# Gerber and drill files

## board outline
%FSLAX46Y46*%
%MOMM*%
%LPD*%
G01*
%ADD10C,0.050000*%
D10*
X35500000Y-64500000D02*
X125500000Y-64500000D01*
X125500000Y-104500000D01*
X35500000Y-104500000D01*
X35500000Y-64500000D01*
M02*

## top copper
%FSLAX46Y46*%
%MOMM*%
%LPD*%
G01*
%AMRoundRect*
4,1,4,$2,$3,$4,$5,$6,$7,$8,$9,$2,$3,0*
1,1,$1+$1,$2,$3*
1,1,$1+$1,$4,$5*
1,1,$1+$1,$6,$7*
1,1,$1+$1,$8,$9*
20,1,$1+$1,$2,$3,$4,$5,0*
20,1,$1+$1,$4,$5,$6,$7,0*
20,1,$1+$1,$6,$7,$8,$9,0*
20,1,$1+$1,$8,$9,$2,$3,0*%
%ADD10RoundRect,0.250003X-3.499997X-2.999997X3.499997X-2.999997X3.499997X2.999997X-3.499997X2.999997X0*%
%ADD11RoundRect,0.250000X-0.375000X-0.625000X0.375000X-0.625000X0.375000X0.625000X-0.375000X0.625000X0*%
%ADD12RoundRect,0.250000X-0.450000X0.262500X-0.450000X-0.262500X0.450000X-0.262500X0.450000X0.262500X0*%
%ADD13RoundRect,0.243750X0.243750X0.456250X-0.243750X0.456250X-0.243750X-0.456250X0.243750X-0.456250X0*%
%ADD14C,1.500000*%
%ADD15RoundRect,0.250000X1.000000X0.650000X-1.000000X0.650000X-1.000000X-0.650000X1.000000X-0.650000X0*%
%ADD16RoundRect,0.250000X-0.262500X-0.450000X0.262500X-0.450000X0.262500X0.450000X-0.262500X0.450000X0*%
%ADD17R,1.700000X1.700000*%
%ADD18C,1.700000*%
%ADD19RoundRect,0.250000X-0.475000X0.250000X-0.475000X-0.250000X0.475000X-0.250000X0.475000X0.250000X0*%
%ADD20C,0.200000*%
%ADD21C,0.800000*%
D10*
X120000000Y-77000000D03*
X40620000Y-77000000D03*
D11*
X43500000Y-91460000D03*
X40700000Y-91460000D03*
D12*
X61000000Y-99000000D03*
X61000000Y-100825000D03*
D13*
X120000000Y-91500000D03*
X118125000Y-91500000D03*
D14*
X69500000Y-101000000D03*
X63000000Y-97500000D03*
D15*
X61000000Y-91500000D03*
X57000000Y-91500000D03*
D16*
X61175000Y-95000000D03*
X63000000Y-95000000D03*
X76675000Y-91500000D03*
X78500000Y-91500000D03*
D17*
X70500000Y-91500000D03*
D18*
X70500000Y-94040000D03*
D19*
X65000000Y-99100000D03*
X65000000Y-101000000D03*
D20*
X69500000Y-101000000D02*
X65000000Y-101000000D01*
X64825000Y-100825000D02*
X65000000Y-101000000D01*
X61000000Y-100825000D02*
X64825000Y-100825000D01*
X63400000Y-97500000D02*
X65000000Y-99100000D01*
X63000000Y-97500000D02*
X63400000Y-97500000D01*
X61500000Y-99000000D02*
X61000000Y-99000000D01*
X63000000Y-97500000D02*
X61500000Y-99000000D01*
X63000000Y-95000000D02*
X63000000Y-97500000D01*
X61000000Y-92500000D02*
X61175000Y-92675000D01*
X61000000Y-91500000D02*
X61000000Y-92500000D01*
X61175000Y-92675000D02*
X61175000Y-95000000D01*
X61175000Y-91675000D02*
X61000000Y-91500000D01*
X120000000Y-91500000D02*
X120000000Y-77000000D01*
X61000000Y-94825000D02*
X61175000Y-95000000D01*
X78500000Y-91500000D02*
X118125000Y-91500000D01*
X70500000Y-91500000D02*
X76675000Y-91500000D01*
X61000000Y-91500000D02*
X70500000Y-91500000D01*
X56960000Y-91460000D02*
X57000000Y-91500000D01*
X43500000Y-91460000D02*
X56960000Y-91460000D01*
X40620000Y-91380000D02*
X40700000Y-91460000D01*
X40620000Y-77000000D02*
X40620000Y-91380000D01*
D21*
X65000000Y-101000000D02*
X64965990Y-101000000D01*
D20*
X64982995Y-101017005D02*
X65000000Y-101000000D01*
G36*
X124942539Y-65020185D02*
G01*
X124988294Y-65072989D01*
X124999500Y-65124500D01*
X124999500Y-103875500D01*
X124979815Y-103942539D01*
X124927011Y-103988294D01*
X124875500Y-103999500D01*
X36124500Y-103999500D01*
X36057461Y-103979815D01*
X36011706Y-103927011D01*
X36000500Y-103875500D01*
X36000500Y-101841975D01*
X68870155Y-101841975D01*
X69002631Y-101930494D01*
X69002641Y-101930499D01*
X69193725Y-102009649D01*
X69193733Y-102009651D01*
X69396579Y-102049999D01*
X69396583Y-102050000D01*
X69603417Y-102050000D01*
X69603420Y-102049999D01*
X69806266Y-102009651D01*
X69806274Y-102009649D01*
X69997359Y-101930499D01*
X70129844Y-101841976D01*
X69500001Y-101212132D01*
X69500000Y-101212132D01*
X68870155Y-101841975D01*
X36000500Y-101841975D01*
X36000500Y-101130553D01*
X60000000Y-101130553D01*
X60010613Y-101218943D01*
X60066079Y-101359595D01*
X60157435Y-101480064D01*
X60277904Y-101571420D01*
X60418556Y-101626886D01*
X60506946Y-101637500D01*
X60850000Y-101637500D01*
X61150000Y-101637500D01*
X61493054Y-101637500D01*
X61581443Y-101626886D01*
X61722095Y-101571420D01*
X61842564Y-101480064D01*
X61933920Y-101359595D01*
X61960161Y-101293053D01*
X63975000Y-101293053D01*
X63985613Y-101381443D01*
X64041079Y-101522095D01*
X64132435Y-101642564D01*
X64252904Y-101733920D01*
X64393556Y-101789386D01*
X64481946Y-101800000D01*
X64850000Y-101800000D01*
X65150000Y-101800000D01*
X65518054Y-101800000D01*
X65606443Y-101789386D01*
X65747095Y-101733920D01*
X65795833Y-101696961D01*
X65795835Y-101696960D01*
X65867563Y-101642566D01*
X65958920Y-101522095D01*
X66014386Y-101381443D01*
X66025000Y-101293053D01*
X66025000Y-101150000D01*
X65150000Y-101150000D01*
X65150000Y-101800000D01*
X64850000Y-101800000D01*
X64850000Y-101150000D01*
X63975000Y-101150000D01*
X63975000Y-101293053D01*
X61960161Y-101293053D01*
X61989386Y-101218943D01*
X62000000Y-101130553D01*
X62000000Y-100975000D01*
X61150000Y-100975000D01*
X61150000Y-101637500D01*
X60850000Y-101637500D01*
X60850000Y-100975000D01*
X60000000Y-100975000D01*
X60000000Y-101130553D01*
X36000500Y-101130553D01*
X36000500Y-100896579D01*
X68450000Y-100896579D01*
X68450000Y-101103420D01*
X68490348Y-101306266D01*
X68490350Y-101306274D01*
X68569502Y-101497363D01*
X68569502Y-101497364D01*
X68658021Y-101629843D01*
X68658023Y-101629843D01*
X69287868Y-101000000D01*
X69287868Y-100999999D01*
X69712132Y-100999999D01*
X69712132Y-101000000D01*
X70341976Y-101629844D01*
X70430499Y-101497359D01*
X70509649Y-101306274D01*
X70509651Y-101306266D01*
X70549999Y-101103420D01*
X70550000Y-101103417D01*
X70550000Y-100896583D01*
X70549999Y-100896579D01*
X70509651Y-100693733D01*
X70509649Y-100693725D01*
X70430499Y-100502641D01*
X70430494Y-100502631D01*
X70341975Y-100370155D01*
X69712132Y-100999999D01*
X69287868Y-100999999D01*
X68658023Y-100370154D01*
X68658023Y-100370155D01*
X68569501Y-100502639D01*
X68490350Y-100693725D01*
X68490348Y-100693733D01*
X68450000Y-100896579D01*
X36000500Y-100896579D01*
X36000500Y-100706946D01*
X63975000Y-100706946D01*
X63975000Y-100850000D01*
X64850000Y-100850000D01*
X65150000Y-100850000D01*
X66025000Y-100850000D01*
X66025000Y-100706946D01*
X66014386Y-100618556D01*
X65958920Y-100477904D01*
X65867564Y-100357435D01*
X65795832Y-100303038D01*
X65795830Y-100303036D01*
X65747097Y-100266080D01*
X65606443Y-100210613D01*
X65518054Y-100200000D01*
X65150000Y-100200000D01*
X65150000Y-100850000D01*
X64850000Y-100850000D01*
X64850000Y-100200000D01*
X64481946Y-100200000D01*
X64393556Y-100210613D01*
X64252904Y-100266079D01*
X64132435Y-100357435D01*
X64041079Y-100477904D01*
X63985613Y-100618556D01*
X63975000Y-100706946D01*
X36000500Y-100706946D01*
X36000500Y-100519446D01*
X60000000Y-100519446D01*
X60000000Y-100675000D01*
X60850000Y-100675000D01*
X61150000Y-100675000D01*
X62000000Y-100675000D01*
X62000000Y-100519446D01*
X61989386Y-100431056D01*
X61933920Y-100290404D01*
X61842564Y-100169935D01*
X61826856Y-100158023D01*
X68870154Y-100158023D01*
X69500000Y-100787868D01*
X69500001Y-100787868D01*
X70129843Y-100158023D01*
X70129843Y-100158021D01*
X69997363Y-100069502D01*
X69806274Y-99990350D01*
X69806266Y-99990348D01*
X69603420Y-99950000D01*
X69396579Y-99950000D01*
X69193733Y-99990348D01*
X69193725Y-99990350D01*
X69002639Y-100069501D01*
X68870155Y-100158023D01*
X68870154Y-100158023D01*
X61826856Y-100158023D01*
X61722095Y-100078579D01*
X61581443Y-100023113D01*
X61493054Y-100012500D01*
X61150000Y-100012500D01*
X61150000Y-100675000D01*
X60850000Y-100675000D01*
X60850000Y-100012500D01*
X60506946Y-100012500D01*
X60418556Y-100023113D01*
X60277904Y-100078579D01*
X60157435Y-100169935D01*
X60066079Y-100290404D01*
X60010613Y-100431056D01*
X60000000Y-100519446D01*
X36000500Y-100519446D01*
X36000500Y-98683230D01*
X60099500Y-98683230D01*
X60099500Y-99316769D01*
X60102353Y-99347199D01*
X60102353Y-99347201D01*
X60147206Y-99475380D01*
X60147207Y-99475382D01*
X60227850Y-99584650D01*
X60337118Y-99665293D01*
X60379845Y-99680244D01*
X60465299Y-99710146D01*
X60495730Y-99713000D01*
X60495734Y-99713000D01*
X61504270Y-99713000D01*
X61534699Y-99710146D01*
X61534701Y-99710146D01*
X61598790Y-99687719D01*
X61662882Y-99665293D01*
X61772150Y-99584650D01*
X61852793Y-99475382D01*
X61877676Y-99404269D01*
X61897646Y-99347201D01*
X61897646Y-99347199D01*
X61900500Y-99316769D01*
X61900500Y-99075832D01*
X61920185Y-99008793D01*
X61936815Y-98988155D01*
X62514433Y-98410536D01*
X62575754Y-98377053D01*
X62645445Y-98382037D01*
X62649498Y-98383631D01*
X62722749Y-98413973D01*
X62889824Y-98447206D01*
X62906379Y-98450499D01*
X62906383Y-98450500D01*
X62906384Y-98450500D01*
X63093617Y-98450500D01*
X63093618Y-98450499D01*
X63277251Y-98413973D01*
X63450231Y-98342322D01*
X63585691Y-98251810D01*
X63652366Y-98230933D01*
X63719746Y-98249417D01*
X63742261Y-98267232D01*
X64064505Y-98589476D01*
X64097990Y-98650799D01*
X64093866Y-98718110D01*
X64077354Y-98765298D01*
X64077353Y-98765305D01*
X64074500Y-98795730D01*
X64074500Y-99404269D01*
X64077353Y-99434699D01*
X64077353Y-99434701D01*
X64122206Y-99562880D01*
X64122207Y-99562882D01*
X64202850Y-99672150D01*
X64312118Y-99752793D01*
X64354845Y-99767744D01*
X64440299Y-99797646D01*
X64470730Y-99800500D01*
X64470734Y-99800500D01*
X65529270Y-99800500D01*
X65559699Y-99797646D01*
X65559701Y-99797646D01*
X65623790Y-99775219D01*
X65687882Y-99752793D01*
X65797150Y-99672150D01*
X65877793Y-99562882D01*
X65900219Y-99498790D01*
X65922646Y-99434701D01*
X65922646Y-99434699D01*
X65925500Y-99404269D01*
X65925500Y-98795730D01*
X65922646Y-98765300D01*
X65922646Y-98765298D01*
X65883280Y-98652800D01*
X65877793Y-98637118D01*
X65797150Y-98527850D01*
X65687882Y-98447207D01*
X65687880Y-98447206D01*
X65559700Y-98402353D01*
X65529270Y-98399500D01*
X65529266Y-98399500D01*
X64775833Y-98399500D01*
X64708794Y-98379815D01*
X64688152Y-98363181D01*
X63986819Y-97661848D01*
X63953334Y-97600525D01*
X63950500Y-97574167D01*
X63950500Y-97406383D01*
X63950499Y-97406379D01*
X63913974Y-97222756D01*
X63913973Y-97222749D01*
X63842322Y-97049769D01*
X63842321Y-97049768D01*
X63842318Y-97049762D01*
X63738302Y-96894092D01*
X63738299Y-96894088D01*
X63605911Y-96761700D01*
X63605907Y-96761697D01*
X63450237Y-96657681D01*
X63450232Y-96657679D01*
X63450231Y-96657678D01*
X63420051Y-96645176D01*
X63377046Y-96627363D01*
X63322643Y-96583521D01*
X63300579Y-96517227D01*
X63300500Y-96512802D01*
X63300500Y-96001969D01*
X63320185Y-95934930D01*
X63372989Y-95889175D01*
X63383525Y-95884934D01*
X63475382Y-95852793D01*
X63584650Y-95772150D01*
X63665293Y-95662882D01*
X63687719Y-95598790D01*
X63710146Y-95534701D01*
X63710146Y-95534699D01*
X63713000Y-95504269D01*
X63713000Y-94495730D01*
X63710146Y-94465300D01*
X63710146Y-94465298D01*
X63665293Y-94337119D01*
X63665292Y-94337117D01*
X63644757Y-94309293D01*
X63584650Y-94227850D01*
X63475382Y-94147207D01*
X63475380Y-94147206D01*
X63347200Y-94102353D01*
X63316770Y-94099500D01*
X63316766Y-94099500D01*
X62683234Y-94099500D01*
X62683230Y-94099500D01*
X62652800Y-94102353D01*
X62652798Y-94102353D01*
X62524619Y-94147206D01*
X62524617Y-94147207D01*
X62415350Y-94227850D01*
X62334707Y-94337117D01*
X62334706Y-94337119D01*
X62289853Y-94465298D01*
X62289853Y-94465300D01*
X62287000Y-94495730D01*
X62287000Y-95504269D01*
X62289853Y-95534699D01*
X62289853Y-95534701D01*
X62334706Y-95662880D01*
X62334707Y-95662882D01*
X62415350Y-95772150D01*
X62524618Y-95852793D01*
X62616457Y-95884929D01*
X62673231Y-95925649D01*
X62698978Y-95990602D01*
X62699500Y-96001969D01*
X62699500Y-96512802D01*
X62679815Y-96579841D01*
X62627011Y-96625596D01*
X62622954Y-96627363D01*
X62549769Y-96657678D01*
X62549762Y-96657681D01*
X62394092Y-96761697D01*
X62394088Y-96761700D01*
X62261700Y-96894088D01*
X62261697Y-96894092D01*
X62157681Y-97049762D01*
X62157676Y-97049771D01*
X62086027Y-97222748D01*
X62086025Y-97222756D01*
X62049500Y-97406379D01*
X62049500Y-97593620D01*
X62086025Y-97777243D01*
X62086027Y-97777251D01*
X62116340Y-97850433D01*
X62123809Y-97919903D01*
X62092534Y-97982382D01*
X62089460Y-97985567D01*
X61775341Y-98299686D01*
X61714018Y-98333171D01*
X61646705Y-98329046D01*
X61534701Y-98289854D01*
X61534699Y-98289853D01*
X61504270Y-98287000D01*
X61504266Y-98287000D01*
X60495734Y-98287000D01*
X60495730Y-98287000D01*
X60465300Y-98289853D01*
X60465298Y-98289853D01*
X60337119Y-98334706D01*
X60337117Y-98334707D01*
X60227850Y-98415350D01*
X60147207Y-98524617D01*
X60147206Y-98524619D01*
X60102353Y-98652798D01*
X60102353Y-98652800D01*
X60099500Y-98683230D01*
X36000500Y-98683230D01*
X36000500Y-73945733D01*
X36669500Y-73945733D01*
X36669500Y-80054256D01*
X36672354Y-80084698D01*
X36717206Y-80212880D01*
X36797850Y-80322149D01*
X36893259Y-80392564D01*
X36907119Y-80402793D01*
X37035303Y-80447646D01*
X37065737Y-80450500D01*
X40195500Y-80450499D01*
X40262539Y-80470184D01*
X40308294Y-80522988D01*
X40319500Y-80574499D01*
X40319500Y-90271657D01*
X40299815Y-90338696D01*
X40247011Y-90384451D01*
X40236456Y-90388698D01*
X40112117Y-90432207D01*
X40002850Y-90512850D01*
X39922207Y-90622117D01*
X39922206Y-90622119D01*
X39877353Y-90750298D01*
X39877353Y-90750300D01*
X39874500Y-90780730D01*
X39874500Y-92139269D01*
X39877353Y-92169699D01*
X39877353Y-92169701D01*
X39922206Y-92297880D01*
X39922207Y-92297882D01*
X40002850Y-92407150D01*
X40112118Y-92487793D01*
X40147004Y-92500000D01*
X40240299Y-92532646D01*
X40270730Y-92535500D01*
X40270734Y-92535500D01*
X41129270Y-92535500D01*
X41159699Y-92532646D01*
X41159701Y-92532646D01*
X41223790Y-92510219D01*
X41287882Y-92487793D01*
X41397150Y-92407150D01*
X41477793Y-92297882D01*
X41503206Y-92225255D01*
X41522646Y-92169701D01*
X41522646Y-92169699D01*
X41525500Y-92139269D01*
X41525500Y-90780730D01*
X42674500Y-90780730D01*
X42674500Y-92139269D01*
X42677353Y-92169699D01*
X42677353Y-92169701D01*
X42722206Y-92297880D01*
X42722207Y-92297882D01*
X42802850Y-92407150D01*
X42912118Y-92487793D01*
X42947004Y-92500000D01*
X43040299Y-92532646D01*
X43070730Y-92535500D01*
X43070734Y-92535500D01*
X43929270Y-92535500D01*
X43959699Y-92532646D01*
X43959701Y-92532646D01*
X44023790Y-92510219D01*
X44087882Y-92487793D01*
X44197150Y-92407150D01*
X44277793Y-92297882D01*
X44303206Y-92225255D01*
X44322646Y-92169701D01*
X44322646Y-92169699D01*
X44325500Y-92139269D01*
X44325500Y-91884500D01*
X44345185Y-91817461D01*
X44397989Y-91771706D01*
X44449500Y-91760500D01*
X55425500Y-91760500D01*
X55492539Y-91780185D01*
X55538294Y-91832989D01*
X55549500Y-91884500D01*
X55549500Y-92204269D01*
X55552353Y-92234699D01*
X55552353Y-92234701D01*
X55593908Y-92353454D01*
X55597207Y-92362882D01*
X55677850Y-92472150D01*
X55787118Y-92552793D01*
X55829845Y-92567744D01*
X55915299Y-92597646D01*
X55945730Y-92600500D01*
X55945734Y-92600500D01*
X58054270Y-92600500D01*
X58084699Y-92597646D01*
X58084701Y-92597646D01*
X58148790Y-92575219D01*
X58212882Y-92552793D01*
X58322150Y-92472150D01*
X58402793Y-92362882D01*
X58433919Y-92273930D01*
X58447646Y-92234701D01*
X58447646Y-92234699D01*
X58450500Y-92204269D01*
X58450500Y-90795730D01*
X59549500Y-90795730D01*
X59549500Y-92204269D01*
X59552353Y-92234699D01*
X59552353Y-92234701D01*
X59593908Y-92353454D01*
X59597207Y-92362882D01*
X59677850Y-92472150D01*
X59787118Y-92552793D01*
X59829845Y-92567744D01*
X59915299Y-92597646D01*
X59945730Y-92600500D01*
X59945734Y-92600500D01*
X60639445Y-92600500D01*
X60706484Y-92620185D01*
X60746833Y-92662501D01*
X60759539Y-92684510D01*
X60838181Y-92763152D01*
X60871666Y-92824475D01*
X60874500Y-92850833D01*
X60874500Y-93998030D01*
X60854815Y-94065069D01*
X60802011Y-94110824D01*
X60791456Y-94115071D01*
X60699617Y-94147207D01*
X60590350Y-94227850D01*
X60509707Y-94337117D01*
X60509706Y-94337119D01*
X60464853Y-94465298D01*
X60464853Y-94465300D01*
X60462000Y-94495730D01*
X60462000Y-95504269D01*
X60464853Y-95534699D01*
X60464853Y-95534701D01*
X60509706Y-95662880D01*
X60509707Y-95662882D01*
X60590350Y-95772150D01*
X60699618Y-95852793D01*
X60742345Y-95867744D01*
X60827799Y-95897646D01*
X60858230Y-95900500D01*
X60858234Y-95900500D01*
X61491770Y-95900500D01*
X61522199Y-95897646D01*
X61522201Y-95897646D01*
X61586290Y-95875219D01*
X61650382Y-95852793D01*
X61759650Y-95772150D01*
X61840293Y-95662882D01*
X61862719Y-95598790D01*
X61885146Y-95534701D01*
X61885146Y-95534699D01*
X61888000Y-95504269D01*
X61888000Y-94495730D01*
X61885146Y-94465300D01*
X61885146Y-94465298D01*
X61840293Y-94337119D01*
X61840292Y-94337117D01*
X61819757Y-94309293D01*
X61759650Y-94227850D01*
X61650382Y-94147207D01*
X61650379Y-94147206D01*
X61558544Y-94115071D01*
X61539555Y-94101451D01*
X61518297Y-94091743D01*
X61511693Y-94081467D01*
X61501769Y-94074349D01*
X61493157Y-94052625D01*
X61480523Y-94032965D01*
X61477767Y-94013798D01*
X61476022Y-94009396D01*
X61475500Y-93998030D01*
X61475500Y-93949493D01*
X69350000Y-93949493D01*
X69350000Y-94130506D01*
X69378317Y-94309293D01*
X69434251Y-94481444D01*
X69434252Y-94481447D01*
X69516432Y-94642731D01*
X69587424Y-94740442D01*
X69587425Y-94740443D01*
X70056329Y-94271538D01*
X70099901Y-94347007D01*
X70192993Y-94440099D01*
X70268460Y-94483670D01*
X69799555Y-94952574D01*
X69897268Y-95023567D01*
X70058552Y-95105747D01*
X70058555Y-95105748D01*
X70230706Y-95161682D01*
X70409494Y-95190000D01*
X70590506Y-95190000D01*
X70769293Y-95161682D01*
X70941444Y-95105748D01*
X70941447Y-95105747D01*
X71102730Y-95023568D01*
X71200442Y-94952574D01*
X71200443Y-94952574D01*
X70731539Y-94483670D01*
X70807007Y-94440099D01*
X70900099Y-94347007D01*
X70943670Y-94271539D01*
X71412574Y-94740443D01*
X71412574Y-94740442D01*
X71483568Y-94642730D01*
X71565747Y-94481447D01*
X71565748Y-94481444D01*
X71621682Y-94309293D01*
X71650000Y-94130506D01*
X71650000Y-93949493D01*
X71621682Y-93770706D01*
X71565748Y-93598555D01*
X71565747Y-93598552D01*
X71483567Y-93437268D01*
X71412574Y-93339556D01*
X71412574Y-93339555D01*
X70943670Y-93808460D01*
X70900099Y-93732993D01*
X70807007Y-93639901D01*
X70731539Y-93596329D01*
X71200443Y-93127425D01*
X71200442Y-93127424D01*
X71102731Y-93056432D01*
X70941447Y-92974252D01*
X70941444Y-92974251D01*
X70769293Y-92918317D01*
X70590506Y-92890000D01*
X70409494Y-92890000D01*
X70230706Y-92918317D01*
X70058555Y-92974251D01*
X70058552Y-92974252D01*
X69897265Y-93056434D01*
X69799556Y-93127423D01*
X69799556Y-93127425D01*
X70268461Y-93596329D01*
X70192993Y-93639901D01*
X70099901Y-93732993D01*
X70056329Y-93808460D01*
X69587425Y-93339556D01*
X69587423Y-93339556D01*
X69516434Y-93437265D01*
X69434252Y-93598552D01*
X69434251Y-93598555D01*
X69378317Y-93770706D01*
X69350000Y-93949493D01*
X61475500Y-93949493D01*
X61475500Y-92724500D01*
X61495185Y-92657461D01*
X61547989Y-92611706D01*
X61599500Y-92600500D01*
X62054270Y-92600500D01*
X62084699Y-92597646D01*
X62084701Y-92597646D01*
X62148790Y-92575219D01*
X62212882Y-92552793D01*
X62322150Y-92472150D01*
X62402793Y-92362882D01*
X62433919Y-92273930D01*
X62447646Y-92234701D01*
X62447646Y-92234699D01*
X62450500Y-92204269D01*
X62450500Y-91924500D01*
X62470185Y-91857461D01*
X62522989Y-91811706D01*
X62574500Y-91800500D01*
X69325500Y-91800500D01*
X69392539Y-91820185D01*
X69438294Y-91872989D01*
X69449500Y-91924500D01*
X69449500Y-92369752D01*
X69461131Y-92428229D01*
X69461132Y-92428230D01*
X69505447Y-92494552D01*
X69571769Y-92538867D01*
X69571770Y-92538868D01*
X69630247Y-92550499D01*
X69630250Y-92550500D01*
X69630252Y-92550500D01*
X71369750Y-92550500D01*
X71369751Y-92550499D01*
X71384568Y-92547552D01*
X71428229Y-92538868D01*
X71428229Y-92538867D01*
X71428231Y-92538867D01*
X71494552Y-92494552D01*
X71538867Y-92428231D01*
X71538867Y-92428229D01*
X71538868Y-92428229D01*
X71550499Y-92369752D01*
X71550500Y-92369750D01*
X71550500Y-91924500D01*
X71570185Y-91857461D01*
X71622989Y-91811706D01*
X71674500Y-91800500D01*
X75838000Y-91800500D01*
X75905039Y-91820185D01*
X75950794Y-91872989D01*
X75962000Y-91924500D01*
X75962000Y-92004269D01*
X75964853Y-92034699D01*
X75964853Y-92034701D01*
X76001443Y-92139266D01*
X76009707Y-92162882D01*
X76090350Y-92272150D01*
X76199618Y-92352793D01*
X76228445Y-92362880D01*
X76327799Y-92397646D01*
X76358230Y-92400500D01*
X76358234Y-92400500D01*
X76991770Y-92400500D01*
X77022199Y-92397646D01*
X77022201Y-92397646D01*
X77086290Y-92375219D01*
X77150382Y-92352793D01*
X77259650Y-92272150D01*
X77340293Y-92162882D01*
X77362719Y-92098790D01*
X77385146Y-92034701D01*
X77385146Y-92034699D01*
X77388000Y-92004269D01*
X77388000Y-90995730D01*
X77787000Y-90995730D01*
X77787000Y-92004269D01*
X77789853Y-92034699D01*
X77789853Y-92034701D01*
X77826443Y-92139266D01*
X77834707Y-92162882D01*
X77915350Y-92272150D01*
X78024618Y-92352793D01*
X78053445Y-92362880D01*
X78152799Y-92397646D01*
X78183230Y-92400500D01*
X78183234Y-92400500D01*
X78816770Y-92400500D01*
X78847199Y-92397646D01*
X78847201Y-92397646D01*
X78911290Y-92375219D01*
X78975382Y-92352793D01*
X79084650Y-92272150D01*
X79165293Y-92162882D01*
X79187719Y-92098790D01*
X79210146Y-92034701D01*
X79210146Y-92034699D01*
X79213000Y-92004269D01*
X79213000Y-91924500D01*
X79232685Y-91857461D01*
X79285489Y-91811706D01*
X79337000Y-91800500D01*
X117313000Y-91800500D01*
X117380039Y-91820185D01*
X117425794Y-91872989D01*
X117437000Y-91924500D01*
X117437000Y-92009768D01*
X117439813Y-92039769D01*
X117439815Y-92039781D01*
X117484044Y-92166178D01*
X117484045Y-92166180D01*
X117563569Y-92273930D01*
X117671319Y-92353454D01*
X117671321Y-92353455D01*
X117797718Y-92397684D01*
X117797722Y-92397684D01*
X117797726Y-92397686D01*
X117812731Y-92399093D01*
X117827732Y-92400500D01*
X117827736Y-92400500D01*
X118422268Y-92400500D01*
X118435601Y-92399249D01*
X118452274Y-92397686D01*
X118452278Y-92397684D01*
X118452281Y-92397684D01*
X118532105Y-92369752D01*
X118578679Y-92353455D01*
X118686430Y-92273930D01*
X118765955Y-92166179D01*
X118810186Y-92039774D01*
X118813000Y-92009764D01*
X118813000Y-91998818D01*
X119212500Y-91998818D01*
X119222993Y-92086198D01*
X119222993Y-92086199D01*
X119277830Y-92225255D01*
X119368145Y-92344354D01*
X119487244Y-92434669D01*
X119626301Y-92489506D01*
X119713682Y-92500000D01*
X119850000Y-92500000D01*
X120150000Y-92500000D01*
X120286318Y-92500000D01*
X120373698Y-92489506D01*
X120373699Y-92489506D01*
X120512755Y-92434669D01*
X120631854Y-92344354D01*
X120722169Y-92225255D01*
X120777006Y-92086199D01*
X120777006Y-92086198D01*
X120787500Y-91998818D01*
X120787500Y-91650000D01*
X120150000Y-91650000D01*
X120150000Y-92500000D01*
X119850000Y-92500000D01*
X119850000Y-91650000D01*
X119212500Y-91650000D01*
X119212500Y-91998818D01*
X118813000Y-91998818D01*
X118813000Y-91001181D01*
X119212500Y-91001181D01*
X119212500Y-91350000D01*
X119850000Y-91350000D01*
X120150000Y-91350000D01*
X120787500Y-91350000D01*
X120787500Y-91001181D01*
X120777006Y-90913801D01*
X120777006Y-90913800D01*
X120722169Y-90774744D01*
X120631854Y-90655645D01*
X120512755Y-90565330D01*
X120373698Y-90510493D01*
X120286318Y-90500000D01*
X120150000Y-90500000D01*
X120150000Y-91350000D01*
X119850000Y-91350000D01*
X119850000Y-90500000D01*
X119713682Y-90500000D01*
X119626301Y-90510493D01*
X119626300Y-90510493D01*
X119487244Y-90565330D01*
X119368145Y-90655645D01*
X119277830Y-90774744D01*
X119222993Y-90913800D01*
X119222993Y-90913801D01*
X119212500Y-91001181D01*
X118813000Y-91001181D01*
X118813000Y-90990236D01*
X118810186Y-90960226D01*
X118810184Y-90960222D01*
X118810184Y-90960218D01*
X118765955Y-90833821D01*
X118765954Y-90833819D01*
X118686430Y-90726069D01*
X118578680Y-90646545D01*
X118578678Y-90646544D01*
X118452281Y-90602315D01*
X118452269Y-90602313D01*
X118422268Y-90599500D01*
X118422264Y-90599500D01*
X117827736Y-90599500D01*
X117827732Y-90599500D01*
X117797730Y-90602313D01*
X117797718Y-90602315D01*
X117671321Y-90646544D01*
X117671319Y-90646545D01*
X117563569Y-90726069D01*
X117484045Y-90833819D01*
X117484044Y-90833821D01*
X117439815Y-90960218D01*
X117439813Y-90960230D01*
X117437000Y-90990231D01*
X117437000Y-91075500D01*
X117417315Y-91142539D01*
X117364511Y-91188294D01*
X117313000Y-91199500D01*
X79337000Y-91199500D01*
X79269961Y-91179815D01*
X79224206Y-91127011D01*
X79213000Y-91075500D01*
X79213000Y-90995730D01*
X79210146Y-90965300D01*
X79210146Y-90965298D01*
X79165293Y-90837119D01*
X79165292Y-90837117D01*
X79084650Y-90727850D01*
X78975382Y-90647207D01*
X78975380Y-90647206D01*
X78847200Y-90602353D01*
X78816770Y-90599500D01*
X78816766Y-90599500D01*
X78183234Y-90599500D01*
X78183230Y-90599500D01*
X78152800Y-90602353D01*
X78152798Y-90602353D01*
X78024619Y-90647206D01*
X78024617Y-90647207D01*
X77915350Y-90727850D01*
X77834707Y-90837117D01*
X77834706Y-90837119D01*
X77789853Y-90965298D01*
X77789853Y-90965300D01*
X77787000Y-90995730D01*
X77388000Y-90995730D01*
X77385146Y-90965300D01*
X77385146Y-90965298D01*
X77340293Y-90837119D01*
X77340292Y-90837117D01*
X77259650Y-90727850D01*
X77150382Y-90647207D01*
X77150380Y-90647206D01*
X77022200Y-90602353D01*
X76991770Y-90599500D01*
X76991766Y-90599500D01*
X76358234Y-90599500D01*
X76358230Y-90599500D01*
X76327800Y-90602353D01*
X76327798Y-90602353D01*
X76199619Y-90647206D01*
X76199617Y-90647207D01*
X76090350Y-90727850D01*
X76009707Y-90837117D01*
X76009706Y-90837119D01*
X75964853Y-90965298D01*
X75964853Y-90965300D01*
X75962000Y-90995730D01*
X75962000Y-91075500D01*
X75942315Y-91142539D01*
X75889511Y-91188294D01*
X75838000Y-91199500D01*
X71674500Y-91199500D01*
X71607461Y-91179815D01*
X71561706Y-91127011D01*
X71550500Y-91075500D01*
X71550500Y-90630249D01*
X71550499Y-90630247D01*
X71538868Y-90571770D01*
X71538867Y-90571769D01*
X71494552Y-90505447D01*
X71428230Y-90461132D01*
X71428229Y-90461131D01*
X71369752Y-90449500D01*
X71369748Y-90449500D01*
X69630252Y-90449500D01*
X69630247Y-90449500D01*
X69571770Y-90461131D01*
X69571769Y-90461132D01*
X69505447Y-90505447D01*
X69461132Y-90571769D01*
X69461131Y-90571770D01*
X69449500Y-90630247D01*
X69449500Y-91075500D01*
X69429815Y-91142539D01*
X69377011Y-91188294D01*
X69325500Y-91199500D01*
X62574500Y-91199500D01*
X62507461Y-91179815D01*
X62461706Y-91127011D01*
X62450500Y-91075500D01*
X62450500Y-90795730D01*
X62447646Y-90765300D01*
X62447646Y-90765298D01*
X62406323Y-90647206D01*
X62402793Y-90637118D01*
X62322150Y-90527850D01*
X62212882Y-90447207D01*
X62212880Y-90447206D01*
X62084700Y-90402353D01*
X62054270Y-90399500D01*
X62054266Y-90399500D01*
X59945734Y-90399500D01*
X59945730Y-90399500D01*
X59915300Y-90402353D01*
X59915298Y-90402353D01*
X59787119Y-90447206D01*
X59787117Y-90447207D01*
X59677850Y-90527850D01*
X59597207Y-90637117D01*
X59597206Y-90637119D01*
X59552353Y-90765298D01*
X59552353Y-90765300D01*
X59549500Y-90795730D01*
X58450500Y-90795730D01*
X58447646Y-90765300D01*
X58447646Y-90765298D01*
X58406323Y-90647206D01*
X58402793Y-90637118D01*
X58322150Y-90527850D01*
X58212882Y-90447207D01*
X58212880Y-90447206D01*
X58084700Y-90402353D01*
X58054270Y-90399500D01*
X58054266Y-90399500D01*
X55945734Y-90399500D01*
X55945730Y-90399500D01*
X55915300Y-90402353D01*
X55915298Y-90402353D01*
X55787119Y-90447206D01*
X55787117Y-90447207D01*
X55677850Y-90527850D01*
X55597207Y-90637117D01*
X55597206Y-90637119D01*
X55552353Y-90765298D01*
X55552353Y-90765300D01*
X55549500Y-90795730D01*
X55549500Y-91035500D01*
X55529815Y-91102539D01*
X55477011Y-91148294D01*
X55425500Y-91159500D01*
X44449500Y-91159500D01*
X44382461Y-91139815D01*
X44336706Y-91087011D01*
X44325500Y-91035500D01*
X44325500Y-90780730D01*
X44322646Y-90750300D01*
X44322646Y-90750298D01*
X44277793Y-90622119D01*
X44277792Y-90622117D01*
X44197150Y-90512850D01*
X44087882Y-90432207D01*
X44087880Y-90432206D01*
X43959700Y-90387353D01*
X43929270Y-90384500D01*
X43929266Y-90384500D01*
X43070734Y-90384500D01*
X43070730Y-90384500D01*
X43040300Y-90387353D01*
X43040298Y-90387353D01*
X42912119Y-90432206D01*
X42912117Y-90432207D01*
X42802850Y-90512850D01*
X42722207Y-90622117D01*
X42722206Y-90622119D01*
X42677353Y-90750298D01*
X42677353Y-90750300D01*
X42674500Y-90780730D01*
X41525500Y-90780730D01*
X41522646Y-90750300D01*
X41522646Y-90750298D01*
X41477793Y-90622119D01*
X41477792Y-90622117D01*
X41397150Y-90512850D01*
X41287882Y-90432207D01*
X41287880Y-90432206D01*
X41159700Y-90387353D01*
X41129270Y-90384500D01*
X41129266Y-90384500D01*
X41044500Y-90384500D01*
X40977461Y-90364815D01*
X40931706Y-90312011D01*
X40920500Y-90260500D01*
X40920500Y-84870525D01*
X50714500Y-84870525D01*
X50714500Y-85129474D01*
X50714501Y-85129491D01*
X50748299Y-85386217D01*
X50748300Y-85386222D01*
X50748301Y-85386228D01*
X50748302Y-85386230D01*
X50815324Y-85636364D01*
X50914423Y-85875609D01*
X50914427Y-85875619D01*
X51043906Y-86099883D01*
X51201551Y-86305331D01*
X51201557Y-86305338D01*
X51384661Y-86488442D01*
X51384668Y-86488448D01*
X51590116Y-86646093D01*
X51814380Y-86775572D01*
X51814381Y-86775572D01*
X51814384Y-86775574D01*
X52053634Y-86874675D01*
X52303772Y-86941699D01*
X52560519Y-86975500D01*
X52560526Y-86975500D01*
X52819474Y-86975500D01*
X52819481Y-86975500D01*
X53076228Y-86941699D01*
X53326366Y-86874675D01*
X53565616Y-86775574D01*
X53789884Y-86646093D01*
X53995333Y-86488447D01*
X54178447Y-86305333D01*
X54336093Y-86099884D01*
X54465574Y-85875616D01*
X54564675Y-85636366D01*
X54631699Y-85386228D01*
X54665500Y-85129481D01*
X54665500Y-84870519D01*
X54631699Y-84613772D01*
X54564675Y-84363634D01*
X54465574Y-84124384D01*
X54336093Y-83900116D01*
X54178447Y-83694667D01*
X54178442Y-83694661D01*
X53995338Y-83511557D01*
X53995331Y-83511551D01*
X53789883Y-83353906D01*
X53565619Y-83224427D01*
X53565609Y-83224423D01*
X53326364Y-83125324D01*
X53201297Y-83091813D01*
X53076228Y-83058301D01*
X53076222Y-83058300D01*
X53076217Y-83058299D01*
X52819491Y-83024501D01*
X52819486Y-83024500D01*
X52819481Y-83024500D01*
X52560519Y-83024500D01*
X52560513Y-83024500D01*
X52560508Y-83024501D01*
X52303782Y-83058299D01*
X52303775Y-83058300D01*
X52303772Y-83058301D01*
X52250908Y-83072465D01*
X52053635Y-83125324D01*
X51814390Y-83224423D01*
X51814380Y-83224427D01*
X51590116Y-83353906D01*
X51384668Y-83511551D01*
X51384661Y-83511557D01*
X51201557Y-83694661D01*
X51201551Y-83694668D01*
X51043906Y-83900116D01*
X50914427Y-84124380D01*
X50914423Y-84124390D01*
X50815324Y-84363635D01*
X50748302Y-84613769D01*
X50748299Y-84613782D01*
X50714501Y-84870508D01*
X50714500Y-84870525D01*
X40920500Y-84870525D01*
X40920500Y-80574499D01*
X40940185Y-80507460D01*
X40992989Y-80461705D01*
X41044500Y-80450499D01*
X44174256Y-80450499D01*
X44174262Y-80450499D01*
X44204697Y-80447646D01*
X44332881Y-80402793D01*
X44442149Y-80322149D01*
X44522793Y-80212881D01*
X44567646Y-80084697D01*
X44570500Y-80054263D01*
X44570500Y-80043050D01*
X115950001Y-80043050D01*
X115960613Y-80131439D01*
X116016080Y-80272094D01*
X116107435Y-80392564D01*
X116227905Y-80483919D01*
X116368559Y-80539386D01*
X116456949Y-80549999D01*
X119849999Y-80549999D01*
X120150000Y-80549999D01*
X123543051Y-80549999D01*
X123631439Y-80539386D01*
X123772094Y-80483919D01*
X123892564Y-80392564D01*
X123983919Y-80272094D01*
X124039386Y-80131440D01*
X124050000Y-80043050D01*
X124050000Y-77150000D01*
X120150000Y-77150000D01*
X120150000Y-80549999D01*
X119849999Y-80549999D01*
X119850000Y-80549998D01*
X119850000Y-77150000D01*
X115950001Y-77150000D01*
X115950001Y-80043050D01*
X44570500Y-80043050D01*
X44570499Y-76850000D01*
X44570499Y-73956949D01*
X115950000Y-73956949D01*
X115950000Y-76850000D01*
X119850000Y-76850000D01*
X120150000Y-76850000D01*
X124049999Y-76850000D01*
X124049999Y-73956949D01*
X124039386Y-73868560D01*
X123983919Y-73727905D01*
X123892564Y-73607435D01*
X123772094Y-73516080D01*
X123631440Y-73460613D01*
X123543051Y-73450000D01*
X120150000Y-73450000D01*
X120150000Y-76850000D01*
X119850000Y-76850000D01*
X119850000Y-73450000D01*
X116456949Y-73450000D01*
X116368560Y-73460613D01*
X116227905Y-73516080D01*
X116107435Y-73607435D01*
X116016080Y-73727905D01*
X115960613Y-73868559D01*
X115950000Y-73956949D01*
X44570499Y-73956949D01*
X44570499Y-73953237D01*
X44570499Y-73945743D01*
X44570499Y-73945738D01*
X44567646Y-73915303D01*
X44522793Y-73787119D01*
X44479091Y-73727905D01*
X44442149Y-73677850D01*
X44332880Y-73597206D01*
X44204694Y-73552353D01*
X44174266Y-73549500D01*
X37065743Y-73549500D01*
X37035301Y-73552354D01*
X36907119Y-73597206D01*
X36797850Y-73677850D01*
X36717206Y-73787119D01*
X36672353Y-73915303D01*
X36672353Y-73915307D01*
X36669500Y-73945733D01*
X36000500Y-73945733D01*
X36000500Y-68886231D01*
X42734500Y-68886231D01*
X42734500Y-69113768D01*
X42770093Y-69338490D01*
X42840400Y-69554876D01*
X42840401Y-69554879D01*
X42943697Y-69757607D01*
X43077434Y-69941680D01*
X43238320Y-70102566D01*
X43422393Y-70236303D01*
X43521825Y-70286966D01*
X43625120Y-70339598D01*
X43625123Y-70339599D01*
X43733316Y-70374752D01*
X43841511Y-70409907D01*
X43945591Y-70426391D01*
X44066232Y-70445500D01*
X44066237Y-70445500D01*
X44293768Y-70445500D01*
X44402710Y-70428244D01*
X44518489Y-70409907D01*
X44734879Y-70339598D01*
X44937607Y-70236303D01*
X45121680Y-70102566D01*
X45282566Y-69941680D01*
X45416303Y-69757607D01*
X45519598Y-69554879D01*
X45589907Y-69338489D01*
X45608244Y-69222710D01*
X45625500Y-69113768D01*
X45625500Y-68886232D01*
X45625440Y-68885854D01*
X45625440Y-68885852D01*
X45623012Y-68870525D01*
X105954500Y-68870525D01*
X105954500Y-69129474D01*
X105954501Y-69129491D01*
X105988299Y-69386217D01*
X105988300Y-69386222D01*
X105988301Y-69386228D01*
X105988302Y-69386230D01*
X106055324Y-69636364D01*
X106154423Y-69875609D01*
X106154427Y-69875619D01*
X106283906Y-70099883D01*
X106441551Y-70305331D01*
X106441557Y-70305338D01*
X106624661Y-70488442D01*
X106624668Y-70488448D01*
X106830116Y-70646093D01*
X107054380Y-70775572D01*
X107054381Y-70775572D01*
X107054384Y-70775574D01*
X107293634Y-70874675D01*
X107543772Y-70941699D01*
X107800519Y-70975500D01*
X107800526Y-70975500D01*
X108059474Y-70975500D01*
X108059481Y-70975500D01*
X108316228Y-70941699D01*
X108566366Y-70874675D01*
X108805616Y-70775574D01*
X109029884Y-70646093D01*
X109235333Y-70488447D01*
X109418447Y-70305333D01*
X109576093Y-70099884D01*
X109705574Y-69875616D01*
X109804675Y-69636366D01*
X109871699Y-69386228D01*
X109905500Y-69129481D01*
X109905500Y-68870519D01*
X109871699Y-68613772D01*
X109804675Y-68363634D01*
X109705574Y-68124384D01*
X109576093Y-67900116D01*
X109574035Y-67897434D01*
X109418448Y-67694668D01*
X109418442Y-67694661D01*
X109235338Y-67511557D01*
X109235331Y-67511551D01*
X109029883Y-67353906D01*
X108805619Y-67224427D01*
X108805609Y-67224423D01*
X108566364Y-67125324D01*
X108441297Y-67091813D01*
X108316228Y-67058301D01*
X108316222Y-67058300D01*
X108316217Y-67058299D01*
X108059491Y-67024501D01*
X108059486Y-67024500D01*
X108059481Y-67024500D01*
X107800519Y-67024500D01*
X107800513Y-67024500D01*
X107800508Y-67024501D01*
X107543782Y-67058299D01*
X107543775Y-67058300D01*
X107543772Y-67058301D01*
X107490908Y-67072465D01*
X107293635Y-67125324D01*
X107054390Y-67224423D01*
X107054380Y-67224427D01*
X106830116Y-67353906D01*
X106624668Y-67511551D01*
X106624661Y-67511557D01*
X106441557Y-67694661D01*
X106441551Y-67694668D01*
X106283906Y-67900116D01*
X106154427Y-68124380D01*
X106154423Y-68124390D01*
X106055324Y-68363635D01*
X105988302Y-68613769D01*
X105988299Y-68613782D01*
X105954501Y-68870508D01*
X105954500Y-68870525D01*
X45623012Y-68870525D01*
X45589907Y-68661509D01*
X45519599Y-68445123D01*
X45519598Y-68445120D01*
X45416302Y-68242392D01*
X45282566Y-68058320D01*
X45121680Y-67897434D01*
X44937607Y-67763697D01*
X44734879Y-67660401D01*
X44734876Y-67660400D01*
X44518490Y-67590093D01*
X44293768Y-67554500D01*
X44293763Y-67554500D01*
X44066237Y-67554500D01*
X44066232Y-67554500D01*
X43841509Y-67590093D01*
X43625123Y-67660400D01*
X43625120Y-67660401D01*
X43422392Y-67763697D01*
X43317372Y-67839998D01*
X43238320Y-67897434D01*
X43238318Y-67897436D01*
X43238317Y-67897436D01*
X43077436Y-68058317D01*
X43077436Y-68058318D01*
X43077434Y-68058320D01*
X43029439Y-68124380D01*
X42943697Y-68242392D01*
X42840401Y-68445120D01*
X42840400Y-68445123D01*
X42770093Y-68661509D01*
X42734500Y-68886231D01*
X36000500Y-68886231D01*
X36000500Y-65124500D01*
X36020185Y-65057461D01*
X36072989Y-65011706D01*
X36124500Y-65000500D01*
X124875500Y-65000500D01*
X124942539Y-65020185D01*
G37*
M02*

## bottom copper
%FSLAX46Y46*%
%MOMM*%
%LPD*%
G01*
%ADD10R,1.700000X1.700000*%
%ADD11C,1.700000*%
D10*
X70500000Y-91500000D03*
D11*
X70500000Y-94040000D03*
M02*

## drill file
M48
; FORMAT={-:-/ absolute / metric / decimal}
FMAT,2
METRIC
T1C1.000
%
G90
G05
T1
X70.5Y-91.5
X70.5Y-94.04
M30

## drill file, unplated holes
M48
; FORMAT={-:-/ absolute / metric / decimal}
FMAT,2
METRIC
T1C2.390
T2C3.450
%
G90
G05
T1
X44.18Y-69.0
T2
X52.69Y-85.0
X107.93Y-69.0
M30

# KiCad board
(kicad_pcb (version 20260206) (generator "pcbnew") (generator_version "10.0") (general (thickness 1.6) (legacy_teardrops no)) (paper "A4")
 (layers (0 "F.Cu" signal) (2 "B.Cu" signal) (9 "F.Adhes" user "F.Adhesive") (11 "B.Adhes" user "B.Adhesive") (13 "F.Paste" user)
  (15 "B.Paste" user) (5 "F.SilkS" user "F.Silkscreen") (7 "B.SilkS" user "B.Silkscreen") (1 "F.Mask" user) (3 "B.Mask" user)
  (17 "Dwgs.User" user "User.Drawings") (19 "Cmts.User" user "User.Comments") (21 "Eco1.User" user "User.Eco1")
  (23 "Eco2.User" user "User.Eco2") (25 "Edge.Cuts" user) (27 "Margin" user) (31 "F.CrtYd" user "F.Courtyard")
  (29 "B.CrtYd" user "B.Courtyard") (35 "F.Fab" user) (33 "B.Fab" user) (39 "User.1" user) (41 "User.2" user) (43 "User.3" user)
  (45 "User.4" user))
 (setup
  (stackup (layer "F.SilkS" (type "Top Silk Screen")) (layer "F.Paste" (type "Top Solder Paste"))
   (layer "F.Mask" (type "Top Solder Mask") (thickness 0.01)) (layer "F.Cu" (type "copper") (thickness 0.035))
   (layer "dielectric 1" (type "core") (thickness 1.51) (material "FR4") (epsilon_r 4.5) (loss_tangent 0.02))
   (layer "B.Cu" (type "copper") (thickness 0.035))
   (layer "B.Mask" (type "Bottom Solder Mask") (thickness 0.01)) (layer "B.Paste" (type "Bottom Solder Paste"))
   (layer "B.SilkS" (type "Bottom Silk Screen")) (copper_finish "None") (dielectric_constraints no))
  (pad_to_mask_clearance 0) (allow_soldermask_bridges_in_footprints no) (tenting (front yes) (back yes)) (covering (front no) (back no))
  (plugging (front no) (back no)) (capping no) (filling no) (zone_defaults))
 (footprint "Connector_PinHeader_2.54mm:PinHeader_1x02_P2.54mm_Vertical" (layer "F.Cu") (at 70.5 91.5)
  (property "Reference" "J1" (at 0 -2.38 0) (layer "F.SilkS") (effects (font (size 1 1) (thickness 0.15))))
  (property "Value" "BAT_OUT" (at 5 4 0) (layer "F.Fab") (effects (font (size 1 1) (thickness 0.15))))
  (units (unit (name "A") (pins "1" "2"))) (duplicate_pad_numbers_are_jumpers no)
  (pad "1" thru_hole rect (at 0 0) (size 1.7 1.7) (drill 1) (layers "*.Cu" "*.Mask") (remove_unused_layers no) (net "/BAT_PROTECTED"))
  (pad "2" thru_hole circle (at 0 2.54) (size 1.7 1.7) (drill 1) (layers "*.Cu" "*.Mask") (remove_unused_layers no) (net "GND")))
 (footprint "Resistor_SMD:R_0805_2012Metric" (layer "F.Cu") (at 61 99.9125 -90)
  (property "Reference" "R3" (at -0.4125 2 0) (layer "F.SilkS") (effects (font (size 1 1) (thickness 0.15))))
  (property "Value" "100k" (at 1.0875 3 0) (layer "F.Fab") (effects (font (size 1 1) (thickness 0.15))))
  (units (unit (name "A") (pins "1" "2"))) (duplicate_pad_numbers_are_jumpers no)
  (pad "1" smd roundrect (at -0.9125 0 270) (size 1.025 1.4) (layers "F.Cu" "F.Mask" "F.Paste") (roundrect_rratio 0.243902)
   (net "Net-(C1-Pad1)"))
  (pad "2" smd roundrect (at 0.9125 0 270) (size 1.025 1.4) (layers "F.Cu" "F.Mask" "F.Paste") (roundrect_rratio 0.243902) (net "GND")))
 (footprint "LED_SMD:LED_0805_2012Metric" (layer "F.Cu") (at 119.0625 91.5 180)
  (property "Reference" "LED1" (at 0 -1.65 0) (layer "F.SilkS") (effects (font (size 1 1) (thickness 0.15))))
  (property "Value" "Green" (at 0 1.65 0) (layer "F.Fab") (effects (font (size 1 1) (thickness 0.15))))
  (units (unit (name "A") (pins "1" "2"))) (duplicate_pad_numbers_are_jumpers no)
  (pad "1" smd roundrect (at -0.9375 0 180) (size 0.975 1.4) (layers "F.Cu" "F.Mask" "F.Paste") (roundrect_rratio 0.25) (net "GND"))
  (pad "2" smd roundrect (at 0.9375 0 180) (size 0.975 1.4) (layers "F.Cu" "F.Mask" "F.Paste") (roundrect_rratio 0.25) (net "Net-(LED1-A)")))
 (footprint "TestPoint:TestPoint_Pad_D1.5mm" (layer "F.Cu") (at 69.5 101)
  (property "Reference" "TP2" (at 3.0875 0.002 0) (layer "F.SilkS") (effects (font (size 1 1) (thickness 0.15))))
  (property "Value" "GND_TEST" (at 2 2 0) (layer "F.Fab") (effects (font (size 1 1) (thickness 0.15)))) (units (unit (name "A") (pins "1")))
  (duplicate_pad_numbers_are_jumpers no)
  (pad "1" smd circle (at 0 0) (size 1.5 1.5) (layers "F.Cu" "F.Mask") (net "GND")))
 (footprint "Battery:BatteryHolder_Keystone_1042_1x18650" (layer "F.Cu") (at 80.31 77)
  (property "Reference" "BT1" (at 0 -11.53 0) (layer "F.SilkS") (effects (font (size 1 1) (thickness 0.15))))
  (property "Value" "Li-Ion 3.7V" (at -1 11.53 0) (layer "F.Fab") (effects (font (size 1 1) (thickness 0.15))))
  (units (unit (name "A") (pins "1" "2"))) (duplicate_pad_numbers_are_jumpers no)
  (pad "" np_thru_hole circle (at -36.13 -8) (size 2.39 2.39) (drill 2.39) (layers "*.Cu" "*.Mask"))
  (pad "" np_thru_hole circle (at -27.62 8) (size 3.45 3.45) (drill 3.45) (layers "*.Cu" "*.Mask"))
  (pad "" np_thru_hole circle (at 27.62 -8) (size 3.45 3.45) (drill 3.45) (layers "*.Cu" "*.Mask"))
  (pad "1" smd roundrect (at -39.69 0) (size 7.5 6.5) (layers "F.Cu" "F.Mask" "F.Paste") (roundrect_rratio 0.038462) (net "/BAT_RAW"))
  (pad "2" smd roundrect (at 39.69 0) (size 7.5 6.5) (layers "F.Cu" "F.Mask" "F.Paste") (roundrect_rratio 0.038462) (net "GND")))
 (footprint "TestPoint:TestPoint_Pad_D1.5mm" (layer "F.Cu") (at 63 97.5)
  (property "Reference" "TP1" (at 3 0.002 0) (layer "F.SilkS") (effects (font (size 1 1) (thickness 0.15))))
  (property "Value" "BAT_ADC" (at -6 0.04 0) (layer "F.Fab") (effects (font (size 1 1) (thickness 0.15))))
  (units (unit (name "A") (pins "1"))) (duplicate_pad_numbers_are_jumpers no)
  (pad "1" smd circle (at 0 0) (size 1.5 1.5) (layers "F.Cu" "F.Mask") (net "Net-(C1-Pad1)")))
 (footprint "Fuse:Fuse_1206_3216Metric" (layer "F.Cu") (at 42.1 91.46)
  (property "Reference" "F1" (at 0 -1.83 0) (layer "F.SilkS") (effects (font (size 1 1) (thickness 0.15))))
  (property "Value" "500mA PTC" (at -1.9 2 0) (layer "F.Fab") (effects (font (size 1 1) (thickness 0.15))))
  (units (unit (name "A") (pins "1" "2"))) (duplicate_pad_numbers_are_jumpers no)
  (pad "1" smd roundrect (at -1.4 0) (size 1.25 1.75) (layers "F.Cu" "F.Mask" "F.Paste") (roundrect_rratio 0.2) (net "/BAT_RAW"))
  (pad "2" smd roundrect (at 1.4 0) (size 1.25 1.75) (layers "F.Cu" "F.Mask" "F.Paste") (roundrect_rratio 0.2) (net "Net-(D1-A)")))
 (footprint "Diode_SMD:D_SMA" (layer "F.Cu") (at 59 91.5 180)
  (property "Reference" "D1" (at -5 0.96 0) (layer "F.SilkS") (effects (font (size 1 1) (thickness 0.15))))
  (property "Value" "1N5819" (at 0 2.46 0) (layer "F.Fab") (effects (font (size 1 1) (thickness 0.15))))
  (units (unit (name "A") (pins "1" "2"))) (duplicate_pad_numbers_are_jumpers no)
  (pad "1" smd roundrect (at -2 0 180) (size 2.5 1.8) (layers "F.Cu" "F.Mask" "F.Paste") (roundrect_rratio 0.1388888889)
   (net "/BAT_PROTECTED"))
  (pad "2" smd roundrect (at 2 0 180) (size 2.5 1.8) (layers "F.Cu" "F.Mask" "F.Paste") (roundrect_rratio 0.1388888889) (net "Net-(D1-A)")))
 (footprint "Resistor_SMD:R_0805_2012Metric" (layer "F.Cu") (at 62.0875 95)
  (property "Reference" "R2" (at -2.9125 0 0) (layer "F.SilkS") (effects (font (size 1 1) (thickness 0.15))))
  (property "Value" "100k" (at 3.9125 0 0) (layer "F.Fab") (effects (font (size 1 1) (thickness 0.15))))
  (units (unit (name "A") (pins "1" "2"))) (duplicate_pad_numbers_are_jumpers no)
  (pad "1" smd roundrect (at -0.9125 0) (size 1.025 1.4) (layers "F.Cu" "F.Mask" "F.Paste") (roundrect_rratio 0.243902)
   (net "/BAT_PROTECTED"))
  (pad "2" smd roundrect (at 0.9125 0) (size 1.025 1.4) (layers "F.Cu" "F.Mask" "F.Paste") (roundrect_rratio 0.243902) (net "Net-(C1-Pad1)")))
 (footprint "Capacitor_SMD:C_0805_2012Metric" (layer "F.Cu") (at 65 100.05 -90)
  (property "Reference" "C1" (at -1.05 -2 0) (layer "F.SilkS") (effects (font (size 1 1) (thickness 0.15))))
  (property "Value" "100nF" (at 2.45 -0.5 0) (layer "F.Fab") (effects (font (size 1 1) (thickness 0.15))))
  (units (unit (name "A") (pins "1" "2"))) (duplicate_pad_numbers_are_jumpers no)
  (pad "1" smd roundrect (at -0.95 0 270) (size 1 1.45) (layers "F.Cu" "F.Mask" "F.Paste") (roundrect_rratio 0.25) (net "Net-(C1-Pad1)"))
  (pad "2" smd roundrect (at 0.95 0 270) (size 1 1.45) (layers "F.Cu" "F.Mask" "F.Paste") (roundrect_rratio 0.25) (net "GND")))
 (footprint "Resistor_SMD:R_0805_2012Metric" (layer "F.Cu") (at 77.5875 91.5)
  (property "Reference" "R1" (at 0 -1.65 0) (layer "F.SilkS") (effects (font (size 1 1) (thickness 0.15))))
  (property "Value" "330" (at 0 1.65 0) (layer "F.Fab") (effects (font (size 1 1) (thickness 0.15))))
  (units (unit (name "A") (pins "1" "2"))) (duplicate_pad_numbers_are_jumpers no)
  (pad "1" smd roundrect (at -0.9125 0) (size 1.025 1.4) (layers "F.Cu" "F.Mask" "F.Paste") (roundrect_rratio 0.243902)
   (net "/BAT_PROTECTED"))
  (pad "2" smd roundrect (at 0.9125 0) (size 1.025 1.4) (layers "F.Cu" "F.Mask" "F.Paste") (roundrect_rratio 0.243902) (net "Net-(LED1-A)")))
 (gr_rect (start 35.5 64.5) (end 125.5 104.5) (stroke (width 0.05) (type default)) (fill no) (layer "Edge.Cuts"))
 (segment (start 61 91.5) (end 61 92.5) (width 0.2) (layer "F.Cu") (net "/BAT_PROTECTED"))
 (segment (start 61 92.5) (end 61.175 92.675) (width 0.2) (layer "F.Cu") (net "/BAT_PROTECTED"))
 (segment (start 61 94.825) (end 61.175 95) (width 0.2) (layer "F.Cu") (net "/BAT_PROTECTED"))
 (segment (start 61.175 92.675) (end 61.175 95) (width 0.2) (layer "F.Cu") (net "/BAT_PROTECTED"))
 (segment (start 61.175 91.675) (end 61 91.5) (width 0.2) (layer "F.Cu") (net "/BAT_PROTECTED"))
 (segment (start 70.5 91.5) (end 76.675 91.5) (width 0.2) (layer "F.Cu") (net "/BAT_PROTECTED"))
 (segment (start 61 91.5) (end 70.5 91.5) (width 0.2) (layer "F.Cu") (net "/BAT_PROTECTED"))
 (segment (start 64.825 100.825) (end 65 101) (width 0.2) (layer "F.Cu") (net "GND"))
 (segment (start 64.982995 101.017005) (end 65 101) (width 0.2) (layer "F.Cu") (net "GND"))
 (segment (start 61 100.825) (end 64.825 100.825) (width 0.2) (layer "F.Cu") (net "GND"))
 (segment (start 69.5 101) (end 65 101) (width 0.2) (layer "F.Cu") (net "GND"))
 (segment (start 65 101) (end 64.96599 101) (width 0.8) (layer "F.Cu") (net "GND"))
 (segment (start 120 91.5) (end 120 77) (width 0.2) (layer "F.Cu") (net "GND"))
 (segment (start 63 97.5) (end 63.4 97.5) (width 0.2) (layer "F.Cu") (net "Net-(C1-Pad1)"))
 (segment (start 63 97.5) (end 61.5 99) (width 0.2) (layer "F.Cu") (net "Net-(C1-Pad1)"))
 (segment (start 61.5 99) (end 61 99) (width 0.2) (layer "F.Cu") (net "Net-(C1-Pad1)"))
 (segment (start 63 95) (end 63 97.5) (width 0.2) (layer "F.Cu") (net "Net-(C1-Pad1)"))
 (segment (start 63.4 97.5) (end 65 99.1) (width 0.2) (layer "F.Cu") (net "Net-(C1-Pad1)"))
 (segment (start 78.5 91.5) (end 118.125 91.5) (width 0.2) (layer "F.Cu") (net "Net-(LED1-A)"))
 (segment (start 40.62 91.38) (end 40.7 91.46) (width 0.2) (layer "F.Cu") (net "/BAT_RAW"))
 (segment (start 40.62 77) (end 40.62 91.38) (width 0.2) (layer "F.Cu") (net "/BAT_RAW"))
 (segment (start 43.5 91.46) (end 56.96 91.46) (width 0.2) (layer "F.Cu") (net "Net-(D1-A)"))
 (segment (start 56.96 91.46) (end 57 91.5) (width 0.2) (layer "F.Cu") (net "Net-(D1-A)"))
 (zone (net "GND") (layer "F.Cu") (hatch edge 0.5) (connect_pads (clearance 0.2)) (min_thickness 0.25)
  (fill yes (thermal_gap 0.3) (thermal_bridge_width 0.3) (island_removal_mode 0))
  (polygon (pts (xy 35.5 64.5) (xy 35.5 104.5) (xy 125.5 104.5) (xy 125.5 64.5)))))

